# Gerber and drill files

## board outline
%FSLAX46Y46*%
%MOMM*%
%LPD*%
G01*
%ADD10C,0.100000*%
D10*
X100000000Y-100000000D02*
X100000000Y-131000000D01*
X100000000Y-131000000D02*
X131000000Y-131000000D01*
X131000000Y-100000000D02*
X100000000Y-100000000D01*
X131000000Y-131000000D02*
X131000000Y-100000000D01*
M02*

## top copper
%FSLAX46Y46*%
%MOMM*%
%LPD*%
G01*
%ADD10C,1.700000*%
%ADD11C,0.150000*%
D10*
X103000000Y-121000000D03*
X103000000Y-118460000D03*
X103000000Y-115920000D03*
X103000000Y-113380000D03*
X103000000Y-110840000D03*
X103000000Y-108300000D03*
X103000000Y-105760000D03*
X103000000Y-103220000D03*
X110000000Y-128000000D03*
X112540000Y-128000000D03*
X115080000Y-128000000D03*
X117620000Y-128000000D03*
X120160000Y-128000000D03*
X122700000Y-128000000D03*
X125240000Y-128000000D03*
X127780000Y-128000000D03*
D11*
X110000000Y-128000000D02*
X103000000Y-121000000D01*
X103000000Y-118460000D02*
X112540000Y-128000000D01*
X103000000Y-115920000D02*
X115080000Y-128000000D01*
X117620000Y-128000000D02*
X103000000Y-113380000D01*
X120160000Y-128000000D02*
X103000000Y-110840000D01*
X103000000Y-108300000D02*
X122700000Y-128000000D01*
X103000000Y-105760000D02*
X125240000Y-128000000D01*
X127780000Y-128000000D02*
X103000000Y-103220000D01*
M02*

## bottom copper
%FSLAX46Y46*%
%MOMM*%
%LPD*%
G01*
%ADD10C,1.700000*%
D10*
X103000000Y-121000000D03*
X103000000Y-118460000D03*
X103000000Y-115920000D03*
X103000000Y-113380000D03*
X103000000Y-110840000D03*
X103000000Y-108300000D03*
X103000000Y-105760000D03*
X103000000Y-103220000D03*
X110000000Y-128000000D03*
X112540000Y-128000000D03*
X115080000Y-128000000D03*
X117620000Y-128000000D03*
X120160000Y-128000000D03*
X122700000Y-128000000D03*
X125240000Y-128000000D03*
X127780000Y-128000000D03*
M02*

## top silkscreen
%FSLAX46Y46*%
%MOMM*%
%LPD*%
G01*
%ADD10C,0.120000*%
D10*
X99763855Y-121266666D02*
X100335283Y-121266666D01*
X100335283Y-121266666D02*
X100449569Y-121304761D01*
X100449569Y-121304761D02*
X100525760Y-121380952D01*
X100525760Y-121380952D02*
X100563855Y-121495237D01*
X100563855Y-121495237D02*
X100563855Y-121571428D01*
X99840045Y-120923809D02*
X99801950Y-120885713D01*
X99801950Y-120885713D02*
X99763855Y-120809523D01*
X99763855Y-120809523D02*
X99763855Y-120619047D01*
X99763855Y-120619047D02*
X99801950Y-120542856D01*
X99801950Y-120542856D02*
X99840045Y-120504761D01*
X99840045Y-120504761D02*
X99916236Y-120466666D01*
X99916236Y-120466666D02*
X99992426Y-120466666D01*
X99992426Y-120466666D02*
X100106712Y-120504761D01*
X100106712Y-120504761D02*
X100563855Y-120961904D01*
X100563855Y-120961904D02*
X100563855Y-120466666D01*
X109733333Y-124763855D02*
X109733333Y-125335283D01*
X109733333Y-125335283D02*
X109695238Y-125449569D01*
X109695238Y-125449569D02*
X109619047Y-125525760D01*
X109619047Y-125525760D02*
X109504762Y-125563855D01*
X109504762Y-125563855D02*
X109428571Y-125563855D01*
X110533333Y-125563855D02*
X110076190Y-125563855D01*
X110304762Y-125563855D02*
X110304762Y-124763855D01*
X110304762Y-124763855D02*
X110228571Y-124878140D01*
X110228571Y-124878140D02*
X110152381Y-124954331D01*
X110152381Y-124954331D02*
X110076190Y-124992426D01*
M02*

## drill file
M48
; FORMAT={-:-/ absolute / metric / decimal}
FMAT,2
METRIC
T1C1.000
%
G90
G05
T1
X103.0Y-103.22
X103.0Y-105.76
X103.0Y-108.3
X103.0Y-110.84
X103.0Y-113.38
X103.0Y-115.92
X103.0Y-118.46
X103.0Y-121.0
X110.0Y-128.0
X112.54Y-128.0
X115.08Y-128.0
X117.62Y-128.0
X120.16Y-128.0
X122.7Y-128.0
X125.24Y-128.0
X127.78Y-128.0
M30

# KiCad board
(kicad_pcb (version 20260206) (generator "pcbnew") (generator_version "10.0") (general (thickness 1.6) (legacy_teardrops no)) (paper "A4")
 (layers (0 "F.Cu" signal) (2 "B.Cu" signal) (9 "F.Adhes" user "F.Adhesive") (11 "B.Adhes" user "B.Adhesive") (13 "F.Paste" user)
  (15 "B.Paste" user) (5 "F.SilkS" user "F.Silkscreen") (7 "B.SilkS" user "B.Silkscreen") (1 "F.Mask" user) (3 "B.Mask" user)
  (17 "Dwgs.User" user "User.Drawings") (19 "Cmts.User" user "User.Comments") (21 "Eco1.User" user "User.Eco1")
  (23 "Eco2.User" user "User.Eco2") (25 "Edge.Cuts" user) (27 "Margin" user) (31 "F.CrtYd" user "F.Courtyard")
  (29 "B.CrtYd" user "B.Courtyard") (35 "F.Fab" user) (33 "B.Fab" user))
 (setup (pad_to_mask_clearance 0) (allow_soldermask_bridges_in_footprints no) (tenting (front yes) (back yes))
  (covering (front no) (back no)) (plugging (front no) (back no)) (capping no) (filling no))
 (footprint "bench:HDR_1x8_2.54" (layer "F.Cu") (at 103 121 90)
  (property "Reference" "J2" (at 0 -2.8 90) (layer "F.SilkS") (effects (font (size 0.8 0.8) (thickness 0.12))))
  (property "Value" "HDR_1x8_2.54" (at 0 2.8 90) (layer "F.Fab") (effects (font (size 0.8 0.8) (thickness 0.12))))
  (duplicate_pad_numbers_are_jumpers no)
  (pad "1" thru_hole circle (at 0 0 90) (size 1.7 1.7) (drill 1) (layers "*.Cu" "*.Mask") (remove_unused_layers no) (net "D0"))
  (pad "2" thru_hole circle (at 2.54 0 90) (size 1.7 1.7) (drill 1) (layers "*.Cu" "*.Mask") (remove_unused_layers no) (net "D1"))
  (pad "3" thru_hole circle (at 5.08 0 90) (size 1.7 1.7) (drill 1) (layers "*.Cu" "*.Mask") (remove_unused_layers no) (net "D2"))
  (pad "4" thru_hole circle (at 7.62 0 90) (size 1.7 1.7) (drill 1) (layers "*.Cu" "*.Mask") (remove_unused_layers no) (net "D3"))
  (pad "5" thru_hole circle (at 10.16 0 90) (size 1.7 1.7) (drill 1) (layers "*.Cu" "*.Mask") (remove_unused_layers no) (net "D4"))
  (pad "6" thru_hole circle (at 12.7 0 90) (size 1.7 1.7) (drill 1) (layers "*.Cu" "*.Mask") (remove_unused_layers no) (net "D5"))
  (pad "7" thru_hole circle (at 15.24 0 90) (size 1.7 1.7) (drill 1) (layers "*.Cu" "*.Mask") (remove_unused_layers no) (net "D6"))
  (pad "8" thru_hole circle (at 17.78 0 90) (size 1.7 1.7) (drill 1) (layers "*.Cu" "*.Mask") (remove_unused_layers no) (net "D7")))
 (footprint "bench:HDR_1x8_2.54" (layer "F.Cu") (at 110 128)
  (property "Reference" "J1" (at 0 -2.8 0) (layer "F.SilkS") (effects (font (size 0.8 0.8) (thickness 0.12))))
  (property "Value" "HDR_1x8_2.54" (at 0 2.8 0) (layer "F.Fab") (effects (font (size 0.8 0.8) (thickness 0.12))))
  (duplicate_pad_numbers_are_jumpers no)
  (pad "1" thru_hole circle (at 0 0) (size 1.7 1.7) (drill 1) (layers "*.Cu" "*.Mask") (remove_unused_layers no) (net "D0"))
  (pad "2" thru_hole circle (at 2.54 0) (size 1.7 1.7) (drill 1) (layers "*.Cu" "*.Mask") (remove_unused_layers no) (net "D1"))
  (pad "3" thru_hole circle (at 5.08 0) (size 1.7 1.7) (drill 1) (layers "*.Cu" "*.Mask") (remove_unused_layers no) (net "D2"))
  (pad "4" thru_hole circle (at 7.62 0) (size 1.7 1.7) (drill 1) (layers "*.Cu" "*.Mask") (remove_unused_layers no) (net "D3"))
  (pad "5" thru_hole circle (at 10.16 0) (size 1.7 1.7) (drill 1) (layers "*.Cu" "*.Mask") (remove_unused_layers no) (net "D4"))
  (pad "6" thru_hole circle (at 12.7 0) (size 1.7 1.7) (drill 1) (layers "*.Cu" "*.Mask") (remove_unused_layers no) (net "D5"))
  (pad "7" thru_hole circle (at 15.24 0) (size 1.7 1.7) (drill 1) (layers "*.Cu" "*.Mask") (remove_unused_layers no) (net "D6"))
  (pad "8" thru_hole circle (at 17.78 0) (size 1.7 1.7) (drill 1) (layers "*.Cu" "*.Mask") (remove_unused_layers no) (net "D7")))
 (gr_line (start 100 100) (end 100 131) (stroke (width 0.1) (type solid)) (layer "Edge.Cuts"))
 (gr_line (start 100 131) (end 131 131) (stroke (width 0.1) (type solid)) (layer "Edge.Cuts"))
 (gr_line (start 131 100) (end 100 100) (stroke (width 0.1) (type solid)) (layer "Edge.Cuts"))
 (gr_line (start 131 131) (end 131 100) (stroke (width 0.1) (type solid)) (layer "Edge.Cuts"))
 (segment (start 110 128) (end 103 121) (width 0.15) (layer "F.Cu") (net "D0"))
 (segment (start 103 118.46) (end 112.54 128) (width 0.15) (layer "F.Cu") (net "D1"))
 (segment (start 103 115.92) (end 115.08 128) (width 0.15) (layer "F.Cu") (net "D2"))
 (segment (start 117.62 128) (end 103 113.38) (width 0.15) (layer "F.Cu") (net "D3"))
 (segment (start 120.16 128) (end 103 110.84) (width 0.15) (layer "F.Cu") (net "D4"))
 (segment (start 103 108.3) (end 122.7 128) (width 0.15) (layer "F.Cu") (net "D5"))
 (segment (start 103 105.76) (end 125.24 128) (width 0.15) (layer "F.Cu") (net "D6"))
 (segment (start 127.78 128) (end 103 103.22) (width 0.15) (layer "F.Cu") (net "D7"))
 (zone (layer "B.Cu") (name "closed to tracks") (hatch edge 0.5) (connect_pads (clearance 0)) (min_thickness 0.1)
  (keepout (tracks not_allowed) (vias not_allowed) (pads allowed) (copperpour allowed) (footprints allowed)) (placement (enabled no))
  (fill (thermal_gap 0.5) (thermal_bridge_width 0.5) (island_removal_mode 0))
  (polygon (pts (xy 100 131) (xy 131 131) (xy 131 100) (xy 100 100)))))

